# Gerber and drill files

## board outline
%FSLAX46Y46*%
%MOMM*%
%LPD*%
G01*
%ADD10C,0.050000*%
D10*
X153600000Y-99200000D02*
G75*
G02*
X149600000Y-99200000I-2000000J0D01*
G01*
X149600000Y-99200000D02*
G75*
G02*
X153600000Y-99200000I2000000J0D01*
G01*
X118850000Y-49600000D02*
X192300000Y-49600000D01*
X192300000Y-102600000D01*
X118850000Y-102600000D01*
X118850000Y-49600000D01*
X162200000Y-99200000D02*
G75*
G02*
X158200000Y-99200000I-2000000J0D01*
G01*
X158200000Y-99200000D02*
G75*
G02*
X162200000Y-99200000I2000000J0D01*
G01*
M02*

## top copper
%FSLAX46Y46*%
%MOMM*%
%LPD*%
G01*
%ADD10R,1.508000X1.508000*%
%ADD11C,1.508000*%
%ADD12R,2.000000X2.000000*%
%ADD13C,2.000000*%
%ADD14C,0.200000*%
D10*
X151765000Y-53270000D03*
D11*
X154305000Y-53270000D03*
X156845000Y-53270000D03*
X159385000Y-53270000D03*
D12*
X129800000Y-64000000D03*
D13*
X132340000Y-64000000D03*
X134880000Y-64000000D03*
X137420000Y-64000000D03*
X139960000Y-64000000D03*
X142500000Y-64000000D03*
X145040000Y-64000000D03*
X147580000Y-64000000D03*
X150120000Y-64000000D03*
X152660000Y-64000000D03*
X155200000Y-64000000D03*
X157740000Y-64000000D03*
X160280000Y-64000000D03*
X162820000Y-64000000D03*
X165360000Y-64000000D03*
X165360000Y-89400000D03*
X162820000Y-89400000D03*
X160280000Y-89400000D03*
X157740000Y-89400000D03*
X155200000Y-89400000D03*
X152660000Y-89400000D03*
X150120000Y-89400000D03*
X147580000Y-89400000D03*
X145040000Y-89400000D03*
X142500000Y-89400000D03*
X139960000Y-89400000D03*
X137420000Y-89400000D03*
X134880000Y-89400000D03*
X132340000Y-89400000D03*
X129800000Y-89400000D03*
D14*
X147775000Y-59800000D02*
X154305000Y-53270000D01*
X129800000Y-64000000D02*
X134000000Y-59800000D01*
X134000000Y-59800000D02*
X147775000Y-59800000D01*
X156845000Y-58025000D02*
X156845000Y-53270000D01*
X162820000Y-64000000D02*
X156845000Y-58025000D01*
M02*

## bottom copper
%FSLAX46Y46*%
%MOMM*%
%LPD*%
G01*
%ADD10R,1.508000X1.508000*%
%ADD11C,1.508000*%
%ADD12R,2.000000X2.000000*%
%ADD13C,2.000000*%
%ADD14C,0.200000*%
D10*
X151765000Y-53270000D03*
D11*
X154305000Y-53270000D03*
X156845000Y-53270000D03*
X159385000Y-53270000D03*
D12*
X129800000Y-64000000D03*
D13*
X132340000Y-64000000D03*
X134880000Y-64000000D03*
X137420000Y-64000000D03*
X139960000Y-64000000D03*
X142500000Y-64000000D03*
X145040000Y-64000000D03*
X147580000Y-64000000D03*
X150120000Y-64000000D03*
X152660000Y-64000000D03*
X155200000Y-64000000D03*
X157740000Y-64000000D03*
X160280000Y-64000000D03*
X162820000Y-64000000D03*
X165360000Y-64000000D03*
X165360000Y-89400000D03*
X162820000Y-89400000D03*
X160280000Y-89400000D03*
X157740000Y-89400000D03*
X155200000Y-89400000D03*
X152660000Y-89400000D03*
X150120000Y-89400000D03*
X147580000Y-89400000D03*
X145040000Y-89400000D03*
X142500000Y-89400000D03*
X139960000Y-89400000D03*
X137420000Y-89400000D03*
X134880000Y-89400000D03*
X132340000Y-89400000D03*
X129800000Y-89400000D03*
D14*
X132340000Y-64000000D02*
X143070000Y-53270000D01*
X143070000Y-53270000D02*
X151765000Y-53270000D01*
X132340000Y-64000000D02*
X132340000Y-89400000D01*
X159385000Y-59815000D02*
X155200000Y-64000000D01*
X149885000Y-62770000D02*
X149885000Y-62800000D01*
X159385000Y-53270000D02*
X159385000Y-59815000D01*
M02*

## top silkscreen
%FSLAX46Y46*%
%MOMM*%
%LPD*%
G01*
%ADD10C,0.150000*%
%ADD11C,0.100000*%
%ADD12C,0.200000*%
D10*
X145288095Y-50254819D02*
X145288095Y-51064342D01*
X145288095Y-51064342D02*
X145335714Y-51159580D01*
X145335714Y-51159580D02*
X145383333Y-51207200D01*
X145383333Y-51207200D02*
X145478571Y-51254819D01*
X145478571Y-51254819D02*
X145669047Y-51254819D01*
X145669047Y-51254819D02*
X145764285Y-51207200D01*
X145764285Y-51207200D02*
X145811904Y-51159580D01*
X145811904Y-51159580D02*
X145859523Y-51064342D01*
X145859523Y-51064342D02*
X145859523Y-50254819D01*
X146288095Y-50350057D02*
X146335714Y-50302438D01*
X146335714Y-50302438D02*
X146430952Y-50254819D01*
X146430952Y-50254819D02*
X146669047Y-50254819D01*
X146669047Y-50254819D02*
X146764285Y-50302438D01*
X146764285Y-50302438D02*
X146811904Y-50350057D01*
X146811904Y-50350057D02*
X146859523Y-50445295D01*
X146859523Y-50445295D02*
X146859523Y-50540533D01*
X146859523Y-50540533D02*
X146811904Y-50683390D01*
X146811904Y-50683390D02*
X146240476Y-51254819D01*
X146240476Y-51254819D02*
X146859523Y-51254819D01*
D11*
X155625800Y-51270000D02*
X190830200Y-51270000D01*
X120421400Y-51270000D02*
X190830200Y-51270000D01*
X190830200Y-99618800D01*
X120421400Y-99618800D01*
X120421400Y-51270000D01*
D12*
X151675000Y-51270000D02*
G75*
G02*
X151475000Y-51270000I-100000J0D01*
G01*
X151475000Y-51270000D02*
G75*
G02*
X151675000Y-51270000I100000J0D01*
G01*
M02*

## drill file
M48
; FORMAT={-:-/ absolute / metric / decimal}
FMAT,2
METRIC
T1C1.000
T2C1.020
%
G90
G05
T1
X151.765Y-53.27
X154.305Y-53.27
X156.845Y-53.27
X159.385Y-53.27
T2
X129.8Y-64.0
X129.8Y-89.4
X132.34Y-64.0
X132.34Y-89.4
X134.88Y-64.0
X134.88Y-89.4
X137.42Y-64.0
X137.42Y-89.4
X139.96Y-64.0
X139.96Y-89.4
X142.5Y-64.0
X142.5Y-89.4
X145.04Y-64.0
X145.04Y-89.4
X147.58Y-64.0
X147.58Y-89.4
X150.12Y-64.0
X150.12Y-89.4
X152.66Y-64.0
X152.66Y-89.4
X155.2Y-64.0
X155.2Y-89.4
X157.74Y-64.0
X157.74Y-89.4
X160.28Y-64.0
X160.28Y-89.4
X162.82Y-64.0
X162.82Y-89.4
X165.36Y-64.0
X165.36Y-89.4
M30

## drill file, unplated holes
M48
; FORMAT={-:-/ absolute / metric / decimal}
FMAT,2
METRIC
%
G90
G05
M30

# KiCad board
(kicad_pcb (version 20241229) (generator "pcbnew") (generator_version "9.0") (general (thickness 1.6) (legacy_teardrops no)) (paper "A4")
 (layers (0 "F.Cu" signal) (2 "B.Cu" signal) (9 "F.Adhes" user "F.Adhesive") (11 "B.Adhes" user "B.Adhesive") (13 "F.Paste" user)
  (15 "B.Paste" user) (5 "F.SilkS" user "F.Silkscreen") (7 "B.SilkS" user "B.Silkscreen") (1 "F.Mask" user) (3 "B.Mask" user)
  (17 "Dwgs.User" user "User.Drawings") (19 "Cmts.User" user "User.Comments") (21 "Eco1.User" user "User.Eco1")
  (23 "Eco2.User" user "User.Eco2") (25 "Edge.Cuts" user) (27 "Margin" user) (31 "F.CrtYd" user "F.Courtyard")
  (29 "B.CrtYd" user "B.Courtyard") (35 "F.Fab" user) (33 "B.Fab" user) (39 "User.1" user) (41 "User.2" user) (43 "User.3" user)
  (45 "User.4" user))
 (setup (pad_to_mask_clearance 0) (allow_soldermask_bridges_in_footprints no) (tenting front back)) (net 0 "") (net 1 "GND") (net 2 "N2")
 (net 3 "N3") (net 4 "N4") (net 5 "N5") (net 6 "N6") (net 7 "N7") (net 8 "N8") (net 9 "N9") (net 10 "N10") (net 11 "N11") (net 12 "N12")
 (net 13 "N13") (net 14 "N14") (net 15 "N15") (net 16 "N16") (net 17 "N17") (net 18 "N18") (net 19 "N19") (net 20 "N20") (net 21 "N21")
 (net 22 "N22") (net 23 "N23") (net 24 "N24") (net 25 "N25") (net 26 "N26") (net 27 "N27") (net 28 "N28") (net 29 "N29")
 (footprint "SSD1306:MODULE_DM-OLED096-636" (layer "F.Cu") (at 155.575 64.77)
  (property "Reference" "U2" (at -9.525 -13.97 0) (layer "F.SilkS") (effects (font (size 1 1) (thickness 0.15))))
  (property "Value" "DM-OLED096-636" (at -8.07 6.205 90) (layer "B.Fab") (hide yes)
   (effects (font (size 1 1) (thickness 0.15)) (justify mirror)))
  (fp_line (start 0.0508 -13.5) (end 35.2552 -13.5) (stroke (width 0.1) (type default)) (layer "F.SilkS"))
  (fp_rect (start -35.1536 -13.5) (end 35.2552 34.8488) (stroke (width 0.1) (type default)) (fill no) (layer "F.SilkS"))
  (fp_circle (center -4 -13.5) (end -3.9 -13.5) (stroke (width 0.2) (type solid)) (fill no) (layer "F.SilkS"))
  (pad "1" thru_hole rect (at -3.81 -11.5) (size 1.508 1.508) (drill 1) (layers "*.Cu" "*.Mask") (remove_unused_layers no) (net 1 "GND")
   (solder_mask_margin 0.102))
  (pad "2" thru_hole circle (at -1.27 -11.5) (size 1.508 1.508) (drill 1) (layers "*.Cu" "*.Mask") (remove_unused_layers no) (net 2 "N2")
   (solder_mask_margin 0.102))
  (pad "3" thru_hole circle (at 1.27 -11.5) (size 1.508 1.508) (drill 1) (layers "*.Cu" "*.Mask") (remove_unused_layers no) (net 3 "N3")
   (solder_mask_margin 0.102))
  (pad "4" thru_hole circle (at 3.81 -11.5) (size 1.508 1.508) (drill 1) (layers "*.Cu" "*.Mask") (remove_unused_layers no) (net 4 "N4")
   (solder_mask_margin 0.102)))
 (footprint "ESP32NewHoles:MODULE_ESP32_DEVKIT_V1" (layer "B.Cu") (at 145.315 76.7 -90)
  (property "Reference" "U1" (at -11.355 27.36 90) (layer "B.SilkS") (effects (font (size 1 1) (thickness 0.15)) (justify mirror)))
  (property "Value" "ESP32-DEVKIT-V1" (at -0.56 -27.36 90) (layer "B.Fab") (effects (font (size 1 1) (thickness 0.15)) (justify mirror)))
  (pad "1" thru_hole rect (at -12.7 15.515 270) (size 2 2) (drill 1.02) (layers "*.Cu" "*.Mask") (remove_unused_layers no) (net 2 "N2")
   (solder_mask_margin 0.102))
  (pad "2" thru_hole circle (at -12.7 12.975 270) (size 2 2) (drill 1.02) (layers "*.Cu" "*.Mask") (remove_unused_layers no) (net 1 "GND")
   (solder_mask_margin 0.102))
  (pad "3" thru_hole circle (at -12.7 10.435 270) (size 2 2) (drill 1.02) (layers "*.Cu" "*.Mask") (remove_unused_layers no) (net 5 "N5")
   (solder_mask_margin 0.102))
  (pad "4" thru_hole circle (at -12.7 7.895 270) (size 2 2) (drill 1.02) (layers "*.Cu" "*.Mask") (remove_unused_layers no) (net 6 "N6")
   (solder_mask_margin 0.102))
  (pad "5" thru_hole circle (at -12.7 5.355 270) (size 2 2) (drill 1.02) (layers "*.Cu" "*.Mask") (remove_unused_layers no) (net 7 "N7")
   (solder_mask_margin 0.102))
  (pad "6" thru_hole circle (at -12.7 2.815 270) (size 2 2) (drill 1.02) (layers "*.Cu" "*.Mask") (remove_unused_layers no) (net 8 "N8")
   (solder_mask_margin 0.102))
  (pad "7" thru_hole circle (at -12.7 0.275 270) (size 2 2) (drill 1.02) (layers "*.Cu" "*.Mask") (remove_unused_layers no) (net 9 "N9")
   (solder_mask_margin 0.102))
  (pad "8" thru_hole circle (at -12.7 -2.265 270) (size 2 2) (drill 1.02) (layers "*.Cu" "*.Mask") (remove_unused_layers no) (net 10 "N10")
   (solder_mask_margin 0.102))
  (pad "9" thru_hole circle (at -12.7 -4.805 270) (size 2 2) (drill 1.02) (layers "*.Cu" "*.Mask") (remove_unused_layers no) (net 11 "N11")
   (solder_mask_margin 0.102))
  (pad "10" thru_hole circle (at -12.7 -7.345 270) (size 2 2) (drill 1.02) (layers "*.Cu" "*.Mask") (remove_unused_layers no) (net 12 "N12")
   (solder_mask_margin 0.102))
  (pad "11" thru_hole circle (at -12.7 -9.885 270) (size 2 2) (drill 1.02) (layers "*.Cu" "*.Mask") (remove_unused_layers no) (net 4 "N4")
   (solder_mask_margin 0.102))
  (pad "12" thru_hole circle (at -12.7 -12.425 270) (size 2 2) (drill 1.02) (layers "*.Cu" "*.Mask") (remove_unused_layers no)
   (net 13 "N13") (solder_mask_margin 0.102))
  (pad "13" thru_hole circle (at -12.7 -14.965 270) (size 2 2) (drill 1.02) (layers "*.Cu" "*.Mask") (remove_unused_layers no)
   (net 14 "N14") (solder_mask_margin 0.102))
  (pad "14" thru_hole circle (at -12.7 -17.505 270) (size 2 2) (drill 1.02) (layers "*.Cu" "*.Mask") (remove_unused_layers no) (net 3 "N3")
   (solder_mask_margin 0.102))
  (pad "15" thru_hole circle (at -12.7 -20.045 270) (size 2 2) (drill 1.02) (layers "*.Cu" "*.Mask") (remove_unused_layers no)
   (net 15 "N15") (solder_mask_margin 0.102))
  (pad "16" thru_hole circle (at 12.7 -20.045 270) (size 2 2) (drill 1.02) (layers "*.Cu" "*.Mask") (remove_unused_layers no) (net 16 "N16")
   (solder_mask_margin 0.102))
  (pad "17" thru_hole circle (at 12.7 -17.505 270) (size 2 2) (drill 1.02) (layers "*.Cu" "*.Mask") (remove_unused_layers no) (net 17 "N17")
   (solder_mask_margin 0.102))
  (pad "18" thru_hole circle (at 12.7 -14.965 270) (size 2 2) (drill 1.02) (layers "*.Cu" "*.Mask") (remove_unused_layers no) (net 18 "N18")
   (solder_mask_margin 0.102))
  (pad "19" thru_hole circle (at 12.7 -12.425 270) (size 2 2) (drill 1.02) (layers "*.Cu" "*.Mask") (remove_unused_layers no) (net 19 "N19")
   (solder_mask_margin 0.102))
  (pad "20" thru_hole circle (at 12.7 -9.885 270) (size 2 2) (drill 1.02) (layers "*.Cu" "*.Mask") (remove_unused_layers no) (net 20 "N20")
   (solder_mask_margin 0.102))
  (pad "21" thru_hole circle (at 12.7 -7.345 270) (size 2 2) (drill 1.02) (layers "*.Cu" "*.Mask") (remove_unused_layers no) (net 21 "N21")
   (solder_mask_margin 0.102))
  (pad "22" thru_hole circle (at 12.7 -4.805 270) (size 2 2) (drill 1.02) (layers "*.Cu" "*.Mask") (remove_unused_layers no) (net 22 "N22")
   (solder_mask_margin 0.102))
  (pad "23" thru_hole circle (at 12.7 -2.265 270) (size 2 2) (drill 1.02) (layers "*.Cu" "*.Mask") (remove_unused_layers no) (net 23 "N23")
   (solder_mask_margin 0.102))
  (pad "24" thru_hole circle (at 12.7 0.275 270) (size 2 2) (drill 1.02) (layers "*.Cu" "*.Mask") (remove_unused_layers no) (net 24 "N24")
   (solder_mask_margin 0.102))
  (pad "25" thru_hole circle (at 12.7 2.815 270) (size 2 2) (drill 1.02) (layers "*.Cu" "*.Mask") (remove_unused_layers no) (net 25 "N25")
   (solder_mask_margin 0.102))
  (pad "26" thru_hole circle (at 12.7 5.355 270) (size 2 2) (drill 1.02) (layers "*.Cu" "*.Mask") (remove_unused_layers no) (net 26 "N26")
   (solder_mask_margin 0.102))
  (pad "27" thru_hole circle (at 12.7 7.895 270) (size 2 2) (drill 1.02) (layers "*.Cu" "*.Mask") (remove_unused_layers no) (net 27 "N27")
   (solder_mask_margin 0.102))
  (pad "28" thru_hole circle (at 12.7 10.435 270) (size 2 2) (drill 1.02) (layers "*.Cu" "*.Mask") (remove_unused_layers no) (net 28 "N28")
   (solder_mask_margin 0.102))
  (pad "29" thru_hole circle (at 12.7 12.975 270) (size 2 2) (drill 1.02) (layers "*.Cu" "*.Mask") (remove_unused_layers no) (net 1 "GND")
   (solder_mask_margin 0.102))
  (pad "30" thru_hole circle (at 12.7 15.515 270) (size 2 2) (drill 1.02) (layers "*.Cu" "*.Mask") (remove_unused_layers no) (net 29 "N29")
   (solder_mask_margin 0.102))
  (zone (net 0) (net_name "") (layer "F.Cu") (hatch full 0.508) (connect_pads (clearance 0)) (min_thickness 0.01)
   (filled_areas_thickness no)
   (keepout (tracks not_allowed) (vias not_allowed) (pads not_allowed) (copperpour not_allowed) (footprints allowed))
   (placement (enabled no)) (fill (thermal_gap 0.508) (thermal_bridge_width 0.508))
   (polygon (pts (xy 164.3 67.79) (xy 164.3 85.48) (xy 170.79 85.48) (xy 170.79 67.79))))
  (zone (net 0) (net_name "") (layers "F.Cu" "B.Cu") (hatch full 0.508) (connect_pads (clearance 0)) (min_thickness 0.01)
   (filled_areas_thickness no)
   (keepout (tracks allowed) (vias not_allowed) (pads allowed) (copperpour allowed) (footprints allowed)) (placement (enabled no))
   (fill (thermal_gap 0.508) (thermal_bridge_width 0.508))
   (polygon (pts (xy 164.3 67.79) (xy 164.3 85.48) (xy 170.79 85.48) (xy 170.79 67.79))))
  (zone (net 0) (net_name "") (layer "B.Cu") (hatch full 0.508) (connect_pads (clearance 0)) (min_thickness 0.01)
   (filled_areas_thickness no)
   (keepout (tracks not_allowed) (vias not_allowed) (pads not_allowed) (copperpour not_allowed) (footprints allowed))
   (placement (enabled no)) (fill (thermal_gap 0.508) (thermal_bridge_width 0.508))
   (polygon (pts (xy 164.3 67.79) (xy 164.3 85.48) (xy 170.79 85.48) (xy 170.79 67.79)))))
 (gr_circle (center 151.6 99.2) (end 151.6 97.2) (stroke (width 0.05) (type default)) (fill no) (layer "Edge.Cuts"))
 (gr_rect (start 118.85 49.6) (end 192.3 102.6) (stroke (width 0.05) (type default)) (fill no) (layer "Edge.Cuts"))
 (gr_circle (center 160.2 99.2) (end 160.2 97.2) (stroke (width 0.05) (type default)) (fill no) (layer "Edge.Cuts"))
 (segment (start 132.34 64) (end 143.07 53.27) (width 0.2) (layer "B.Cu") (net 1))
 (segment (start 143.07 53.27) (end 151.765 53.27) (width 0.2) (layer "B.Cu") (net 1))
 (segment (start 132.34 64) (end 132.34 89.4) (width 0.2) (layer "B.Cu") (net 1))
 (segment (start 147.775 59.8) (end 154.305 53.27) (width 0.2) (layer "F.Cu") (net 2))
 (segment (start 129.8 64) (end 134 59.8) (width 0.2) (layer "F.Cu") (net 2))
 (segment (start 134 59.8) (end 147.775 59.8) (width 0.2) (layer "F.Cu") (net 2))
 (segment (start 156.845 58.025) (end 156.845 53.27) (width 0.2) (layer "F.Cu") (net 3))
 (segment (start 162.82 64) (end 156.845 58.025) (width 0.2) (layer "F.Cu") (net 3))
 (segment (start 159.385 59.815) (end 155.2 64) (width 0.2) (layer "B.Cu") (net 4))
 (segment (start 149.885 62.77) (end 149.885 62.8) (width 0.2) (layer "B.Cu") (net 4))
 (segment (start 159.385 53.27) (end 159.385 59.815) (width 0.2) (layer "B.Cu") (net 4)))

